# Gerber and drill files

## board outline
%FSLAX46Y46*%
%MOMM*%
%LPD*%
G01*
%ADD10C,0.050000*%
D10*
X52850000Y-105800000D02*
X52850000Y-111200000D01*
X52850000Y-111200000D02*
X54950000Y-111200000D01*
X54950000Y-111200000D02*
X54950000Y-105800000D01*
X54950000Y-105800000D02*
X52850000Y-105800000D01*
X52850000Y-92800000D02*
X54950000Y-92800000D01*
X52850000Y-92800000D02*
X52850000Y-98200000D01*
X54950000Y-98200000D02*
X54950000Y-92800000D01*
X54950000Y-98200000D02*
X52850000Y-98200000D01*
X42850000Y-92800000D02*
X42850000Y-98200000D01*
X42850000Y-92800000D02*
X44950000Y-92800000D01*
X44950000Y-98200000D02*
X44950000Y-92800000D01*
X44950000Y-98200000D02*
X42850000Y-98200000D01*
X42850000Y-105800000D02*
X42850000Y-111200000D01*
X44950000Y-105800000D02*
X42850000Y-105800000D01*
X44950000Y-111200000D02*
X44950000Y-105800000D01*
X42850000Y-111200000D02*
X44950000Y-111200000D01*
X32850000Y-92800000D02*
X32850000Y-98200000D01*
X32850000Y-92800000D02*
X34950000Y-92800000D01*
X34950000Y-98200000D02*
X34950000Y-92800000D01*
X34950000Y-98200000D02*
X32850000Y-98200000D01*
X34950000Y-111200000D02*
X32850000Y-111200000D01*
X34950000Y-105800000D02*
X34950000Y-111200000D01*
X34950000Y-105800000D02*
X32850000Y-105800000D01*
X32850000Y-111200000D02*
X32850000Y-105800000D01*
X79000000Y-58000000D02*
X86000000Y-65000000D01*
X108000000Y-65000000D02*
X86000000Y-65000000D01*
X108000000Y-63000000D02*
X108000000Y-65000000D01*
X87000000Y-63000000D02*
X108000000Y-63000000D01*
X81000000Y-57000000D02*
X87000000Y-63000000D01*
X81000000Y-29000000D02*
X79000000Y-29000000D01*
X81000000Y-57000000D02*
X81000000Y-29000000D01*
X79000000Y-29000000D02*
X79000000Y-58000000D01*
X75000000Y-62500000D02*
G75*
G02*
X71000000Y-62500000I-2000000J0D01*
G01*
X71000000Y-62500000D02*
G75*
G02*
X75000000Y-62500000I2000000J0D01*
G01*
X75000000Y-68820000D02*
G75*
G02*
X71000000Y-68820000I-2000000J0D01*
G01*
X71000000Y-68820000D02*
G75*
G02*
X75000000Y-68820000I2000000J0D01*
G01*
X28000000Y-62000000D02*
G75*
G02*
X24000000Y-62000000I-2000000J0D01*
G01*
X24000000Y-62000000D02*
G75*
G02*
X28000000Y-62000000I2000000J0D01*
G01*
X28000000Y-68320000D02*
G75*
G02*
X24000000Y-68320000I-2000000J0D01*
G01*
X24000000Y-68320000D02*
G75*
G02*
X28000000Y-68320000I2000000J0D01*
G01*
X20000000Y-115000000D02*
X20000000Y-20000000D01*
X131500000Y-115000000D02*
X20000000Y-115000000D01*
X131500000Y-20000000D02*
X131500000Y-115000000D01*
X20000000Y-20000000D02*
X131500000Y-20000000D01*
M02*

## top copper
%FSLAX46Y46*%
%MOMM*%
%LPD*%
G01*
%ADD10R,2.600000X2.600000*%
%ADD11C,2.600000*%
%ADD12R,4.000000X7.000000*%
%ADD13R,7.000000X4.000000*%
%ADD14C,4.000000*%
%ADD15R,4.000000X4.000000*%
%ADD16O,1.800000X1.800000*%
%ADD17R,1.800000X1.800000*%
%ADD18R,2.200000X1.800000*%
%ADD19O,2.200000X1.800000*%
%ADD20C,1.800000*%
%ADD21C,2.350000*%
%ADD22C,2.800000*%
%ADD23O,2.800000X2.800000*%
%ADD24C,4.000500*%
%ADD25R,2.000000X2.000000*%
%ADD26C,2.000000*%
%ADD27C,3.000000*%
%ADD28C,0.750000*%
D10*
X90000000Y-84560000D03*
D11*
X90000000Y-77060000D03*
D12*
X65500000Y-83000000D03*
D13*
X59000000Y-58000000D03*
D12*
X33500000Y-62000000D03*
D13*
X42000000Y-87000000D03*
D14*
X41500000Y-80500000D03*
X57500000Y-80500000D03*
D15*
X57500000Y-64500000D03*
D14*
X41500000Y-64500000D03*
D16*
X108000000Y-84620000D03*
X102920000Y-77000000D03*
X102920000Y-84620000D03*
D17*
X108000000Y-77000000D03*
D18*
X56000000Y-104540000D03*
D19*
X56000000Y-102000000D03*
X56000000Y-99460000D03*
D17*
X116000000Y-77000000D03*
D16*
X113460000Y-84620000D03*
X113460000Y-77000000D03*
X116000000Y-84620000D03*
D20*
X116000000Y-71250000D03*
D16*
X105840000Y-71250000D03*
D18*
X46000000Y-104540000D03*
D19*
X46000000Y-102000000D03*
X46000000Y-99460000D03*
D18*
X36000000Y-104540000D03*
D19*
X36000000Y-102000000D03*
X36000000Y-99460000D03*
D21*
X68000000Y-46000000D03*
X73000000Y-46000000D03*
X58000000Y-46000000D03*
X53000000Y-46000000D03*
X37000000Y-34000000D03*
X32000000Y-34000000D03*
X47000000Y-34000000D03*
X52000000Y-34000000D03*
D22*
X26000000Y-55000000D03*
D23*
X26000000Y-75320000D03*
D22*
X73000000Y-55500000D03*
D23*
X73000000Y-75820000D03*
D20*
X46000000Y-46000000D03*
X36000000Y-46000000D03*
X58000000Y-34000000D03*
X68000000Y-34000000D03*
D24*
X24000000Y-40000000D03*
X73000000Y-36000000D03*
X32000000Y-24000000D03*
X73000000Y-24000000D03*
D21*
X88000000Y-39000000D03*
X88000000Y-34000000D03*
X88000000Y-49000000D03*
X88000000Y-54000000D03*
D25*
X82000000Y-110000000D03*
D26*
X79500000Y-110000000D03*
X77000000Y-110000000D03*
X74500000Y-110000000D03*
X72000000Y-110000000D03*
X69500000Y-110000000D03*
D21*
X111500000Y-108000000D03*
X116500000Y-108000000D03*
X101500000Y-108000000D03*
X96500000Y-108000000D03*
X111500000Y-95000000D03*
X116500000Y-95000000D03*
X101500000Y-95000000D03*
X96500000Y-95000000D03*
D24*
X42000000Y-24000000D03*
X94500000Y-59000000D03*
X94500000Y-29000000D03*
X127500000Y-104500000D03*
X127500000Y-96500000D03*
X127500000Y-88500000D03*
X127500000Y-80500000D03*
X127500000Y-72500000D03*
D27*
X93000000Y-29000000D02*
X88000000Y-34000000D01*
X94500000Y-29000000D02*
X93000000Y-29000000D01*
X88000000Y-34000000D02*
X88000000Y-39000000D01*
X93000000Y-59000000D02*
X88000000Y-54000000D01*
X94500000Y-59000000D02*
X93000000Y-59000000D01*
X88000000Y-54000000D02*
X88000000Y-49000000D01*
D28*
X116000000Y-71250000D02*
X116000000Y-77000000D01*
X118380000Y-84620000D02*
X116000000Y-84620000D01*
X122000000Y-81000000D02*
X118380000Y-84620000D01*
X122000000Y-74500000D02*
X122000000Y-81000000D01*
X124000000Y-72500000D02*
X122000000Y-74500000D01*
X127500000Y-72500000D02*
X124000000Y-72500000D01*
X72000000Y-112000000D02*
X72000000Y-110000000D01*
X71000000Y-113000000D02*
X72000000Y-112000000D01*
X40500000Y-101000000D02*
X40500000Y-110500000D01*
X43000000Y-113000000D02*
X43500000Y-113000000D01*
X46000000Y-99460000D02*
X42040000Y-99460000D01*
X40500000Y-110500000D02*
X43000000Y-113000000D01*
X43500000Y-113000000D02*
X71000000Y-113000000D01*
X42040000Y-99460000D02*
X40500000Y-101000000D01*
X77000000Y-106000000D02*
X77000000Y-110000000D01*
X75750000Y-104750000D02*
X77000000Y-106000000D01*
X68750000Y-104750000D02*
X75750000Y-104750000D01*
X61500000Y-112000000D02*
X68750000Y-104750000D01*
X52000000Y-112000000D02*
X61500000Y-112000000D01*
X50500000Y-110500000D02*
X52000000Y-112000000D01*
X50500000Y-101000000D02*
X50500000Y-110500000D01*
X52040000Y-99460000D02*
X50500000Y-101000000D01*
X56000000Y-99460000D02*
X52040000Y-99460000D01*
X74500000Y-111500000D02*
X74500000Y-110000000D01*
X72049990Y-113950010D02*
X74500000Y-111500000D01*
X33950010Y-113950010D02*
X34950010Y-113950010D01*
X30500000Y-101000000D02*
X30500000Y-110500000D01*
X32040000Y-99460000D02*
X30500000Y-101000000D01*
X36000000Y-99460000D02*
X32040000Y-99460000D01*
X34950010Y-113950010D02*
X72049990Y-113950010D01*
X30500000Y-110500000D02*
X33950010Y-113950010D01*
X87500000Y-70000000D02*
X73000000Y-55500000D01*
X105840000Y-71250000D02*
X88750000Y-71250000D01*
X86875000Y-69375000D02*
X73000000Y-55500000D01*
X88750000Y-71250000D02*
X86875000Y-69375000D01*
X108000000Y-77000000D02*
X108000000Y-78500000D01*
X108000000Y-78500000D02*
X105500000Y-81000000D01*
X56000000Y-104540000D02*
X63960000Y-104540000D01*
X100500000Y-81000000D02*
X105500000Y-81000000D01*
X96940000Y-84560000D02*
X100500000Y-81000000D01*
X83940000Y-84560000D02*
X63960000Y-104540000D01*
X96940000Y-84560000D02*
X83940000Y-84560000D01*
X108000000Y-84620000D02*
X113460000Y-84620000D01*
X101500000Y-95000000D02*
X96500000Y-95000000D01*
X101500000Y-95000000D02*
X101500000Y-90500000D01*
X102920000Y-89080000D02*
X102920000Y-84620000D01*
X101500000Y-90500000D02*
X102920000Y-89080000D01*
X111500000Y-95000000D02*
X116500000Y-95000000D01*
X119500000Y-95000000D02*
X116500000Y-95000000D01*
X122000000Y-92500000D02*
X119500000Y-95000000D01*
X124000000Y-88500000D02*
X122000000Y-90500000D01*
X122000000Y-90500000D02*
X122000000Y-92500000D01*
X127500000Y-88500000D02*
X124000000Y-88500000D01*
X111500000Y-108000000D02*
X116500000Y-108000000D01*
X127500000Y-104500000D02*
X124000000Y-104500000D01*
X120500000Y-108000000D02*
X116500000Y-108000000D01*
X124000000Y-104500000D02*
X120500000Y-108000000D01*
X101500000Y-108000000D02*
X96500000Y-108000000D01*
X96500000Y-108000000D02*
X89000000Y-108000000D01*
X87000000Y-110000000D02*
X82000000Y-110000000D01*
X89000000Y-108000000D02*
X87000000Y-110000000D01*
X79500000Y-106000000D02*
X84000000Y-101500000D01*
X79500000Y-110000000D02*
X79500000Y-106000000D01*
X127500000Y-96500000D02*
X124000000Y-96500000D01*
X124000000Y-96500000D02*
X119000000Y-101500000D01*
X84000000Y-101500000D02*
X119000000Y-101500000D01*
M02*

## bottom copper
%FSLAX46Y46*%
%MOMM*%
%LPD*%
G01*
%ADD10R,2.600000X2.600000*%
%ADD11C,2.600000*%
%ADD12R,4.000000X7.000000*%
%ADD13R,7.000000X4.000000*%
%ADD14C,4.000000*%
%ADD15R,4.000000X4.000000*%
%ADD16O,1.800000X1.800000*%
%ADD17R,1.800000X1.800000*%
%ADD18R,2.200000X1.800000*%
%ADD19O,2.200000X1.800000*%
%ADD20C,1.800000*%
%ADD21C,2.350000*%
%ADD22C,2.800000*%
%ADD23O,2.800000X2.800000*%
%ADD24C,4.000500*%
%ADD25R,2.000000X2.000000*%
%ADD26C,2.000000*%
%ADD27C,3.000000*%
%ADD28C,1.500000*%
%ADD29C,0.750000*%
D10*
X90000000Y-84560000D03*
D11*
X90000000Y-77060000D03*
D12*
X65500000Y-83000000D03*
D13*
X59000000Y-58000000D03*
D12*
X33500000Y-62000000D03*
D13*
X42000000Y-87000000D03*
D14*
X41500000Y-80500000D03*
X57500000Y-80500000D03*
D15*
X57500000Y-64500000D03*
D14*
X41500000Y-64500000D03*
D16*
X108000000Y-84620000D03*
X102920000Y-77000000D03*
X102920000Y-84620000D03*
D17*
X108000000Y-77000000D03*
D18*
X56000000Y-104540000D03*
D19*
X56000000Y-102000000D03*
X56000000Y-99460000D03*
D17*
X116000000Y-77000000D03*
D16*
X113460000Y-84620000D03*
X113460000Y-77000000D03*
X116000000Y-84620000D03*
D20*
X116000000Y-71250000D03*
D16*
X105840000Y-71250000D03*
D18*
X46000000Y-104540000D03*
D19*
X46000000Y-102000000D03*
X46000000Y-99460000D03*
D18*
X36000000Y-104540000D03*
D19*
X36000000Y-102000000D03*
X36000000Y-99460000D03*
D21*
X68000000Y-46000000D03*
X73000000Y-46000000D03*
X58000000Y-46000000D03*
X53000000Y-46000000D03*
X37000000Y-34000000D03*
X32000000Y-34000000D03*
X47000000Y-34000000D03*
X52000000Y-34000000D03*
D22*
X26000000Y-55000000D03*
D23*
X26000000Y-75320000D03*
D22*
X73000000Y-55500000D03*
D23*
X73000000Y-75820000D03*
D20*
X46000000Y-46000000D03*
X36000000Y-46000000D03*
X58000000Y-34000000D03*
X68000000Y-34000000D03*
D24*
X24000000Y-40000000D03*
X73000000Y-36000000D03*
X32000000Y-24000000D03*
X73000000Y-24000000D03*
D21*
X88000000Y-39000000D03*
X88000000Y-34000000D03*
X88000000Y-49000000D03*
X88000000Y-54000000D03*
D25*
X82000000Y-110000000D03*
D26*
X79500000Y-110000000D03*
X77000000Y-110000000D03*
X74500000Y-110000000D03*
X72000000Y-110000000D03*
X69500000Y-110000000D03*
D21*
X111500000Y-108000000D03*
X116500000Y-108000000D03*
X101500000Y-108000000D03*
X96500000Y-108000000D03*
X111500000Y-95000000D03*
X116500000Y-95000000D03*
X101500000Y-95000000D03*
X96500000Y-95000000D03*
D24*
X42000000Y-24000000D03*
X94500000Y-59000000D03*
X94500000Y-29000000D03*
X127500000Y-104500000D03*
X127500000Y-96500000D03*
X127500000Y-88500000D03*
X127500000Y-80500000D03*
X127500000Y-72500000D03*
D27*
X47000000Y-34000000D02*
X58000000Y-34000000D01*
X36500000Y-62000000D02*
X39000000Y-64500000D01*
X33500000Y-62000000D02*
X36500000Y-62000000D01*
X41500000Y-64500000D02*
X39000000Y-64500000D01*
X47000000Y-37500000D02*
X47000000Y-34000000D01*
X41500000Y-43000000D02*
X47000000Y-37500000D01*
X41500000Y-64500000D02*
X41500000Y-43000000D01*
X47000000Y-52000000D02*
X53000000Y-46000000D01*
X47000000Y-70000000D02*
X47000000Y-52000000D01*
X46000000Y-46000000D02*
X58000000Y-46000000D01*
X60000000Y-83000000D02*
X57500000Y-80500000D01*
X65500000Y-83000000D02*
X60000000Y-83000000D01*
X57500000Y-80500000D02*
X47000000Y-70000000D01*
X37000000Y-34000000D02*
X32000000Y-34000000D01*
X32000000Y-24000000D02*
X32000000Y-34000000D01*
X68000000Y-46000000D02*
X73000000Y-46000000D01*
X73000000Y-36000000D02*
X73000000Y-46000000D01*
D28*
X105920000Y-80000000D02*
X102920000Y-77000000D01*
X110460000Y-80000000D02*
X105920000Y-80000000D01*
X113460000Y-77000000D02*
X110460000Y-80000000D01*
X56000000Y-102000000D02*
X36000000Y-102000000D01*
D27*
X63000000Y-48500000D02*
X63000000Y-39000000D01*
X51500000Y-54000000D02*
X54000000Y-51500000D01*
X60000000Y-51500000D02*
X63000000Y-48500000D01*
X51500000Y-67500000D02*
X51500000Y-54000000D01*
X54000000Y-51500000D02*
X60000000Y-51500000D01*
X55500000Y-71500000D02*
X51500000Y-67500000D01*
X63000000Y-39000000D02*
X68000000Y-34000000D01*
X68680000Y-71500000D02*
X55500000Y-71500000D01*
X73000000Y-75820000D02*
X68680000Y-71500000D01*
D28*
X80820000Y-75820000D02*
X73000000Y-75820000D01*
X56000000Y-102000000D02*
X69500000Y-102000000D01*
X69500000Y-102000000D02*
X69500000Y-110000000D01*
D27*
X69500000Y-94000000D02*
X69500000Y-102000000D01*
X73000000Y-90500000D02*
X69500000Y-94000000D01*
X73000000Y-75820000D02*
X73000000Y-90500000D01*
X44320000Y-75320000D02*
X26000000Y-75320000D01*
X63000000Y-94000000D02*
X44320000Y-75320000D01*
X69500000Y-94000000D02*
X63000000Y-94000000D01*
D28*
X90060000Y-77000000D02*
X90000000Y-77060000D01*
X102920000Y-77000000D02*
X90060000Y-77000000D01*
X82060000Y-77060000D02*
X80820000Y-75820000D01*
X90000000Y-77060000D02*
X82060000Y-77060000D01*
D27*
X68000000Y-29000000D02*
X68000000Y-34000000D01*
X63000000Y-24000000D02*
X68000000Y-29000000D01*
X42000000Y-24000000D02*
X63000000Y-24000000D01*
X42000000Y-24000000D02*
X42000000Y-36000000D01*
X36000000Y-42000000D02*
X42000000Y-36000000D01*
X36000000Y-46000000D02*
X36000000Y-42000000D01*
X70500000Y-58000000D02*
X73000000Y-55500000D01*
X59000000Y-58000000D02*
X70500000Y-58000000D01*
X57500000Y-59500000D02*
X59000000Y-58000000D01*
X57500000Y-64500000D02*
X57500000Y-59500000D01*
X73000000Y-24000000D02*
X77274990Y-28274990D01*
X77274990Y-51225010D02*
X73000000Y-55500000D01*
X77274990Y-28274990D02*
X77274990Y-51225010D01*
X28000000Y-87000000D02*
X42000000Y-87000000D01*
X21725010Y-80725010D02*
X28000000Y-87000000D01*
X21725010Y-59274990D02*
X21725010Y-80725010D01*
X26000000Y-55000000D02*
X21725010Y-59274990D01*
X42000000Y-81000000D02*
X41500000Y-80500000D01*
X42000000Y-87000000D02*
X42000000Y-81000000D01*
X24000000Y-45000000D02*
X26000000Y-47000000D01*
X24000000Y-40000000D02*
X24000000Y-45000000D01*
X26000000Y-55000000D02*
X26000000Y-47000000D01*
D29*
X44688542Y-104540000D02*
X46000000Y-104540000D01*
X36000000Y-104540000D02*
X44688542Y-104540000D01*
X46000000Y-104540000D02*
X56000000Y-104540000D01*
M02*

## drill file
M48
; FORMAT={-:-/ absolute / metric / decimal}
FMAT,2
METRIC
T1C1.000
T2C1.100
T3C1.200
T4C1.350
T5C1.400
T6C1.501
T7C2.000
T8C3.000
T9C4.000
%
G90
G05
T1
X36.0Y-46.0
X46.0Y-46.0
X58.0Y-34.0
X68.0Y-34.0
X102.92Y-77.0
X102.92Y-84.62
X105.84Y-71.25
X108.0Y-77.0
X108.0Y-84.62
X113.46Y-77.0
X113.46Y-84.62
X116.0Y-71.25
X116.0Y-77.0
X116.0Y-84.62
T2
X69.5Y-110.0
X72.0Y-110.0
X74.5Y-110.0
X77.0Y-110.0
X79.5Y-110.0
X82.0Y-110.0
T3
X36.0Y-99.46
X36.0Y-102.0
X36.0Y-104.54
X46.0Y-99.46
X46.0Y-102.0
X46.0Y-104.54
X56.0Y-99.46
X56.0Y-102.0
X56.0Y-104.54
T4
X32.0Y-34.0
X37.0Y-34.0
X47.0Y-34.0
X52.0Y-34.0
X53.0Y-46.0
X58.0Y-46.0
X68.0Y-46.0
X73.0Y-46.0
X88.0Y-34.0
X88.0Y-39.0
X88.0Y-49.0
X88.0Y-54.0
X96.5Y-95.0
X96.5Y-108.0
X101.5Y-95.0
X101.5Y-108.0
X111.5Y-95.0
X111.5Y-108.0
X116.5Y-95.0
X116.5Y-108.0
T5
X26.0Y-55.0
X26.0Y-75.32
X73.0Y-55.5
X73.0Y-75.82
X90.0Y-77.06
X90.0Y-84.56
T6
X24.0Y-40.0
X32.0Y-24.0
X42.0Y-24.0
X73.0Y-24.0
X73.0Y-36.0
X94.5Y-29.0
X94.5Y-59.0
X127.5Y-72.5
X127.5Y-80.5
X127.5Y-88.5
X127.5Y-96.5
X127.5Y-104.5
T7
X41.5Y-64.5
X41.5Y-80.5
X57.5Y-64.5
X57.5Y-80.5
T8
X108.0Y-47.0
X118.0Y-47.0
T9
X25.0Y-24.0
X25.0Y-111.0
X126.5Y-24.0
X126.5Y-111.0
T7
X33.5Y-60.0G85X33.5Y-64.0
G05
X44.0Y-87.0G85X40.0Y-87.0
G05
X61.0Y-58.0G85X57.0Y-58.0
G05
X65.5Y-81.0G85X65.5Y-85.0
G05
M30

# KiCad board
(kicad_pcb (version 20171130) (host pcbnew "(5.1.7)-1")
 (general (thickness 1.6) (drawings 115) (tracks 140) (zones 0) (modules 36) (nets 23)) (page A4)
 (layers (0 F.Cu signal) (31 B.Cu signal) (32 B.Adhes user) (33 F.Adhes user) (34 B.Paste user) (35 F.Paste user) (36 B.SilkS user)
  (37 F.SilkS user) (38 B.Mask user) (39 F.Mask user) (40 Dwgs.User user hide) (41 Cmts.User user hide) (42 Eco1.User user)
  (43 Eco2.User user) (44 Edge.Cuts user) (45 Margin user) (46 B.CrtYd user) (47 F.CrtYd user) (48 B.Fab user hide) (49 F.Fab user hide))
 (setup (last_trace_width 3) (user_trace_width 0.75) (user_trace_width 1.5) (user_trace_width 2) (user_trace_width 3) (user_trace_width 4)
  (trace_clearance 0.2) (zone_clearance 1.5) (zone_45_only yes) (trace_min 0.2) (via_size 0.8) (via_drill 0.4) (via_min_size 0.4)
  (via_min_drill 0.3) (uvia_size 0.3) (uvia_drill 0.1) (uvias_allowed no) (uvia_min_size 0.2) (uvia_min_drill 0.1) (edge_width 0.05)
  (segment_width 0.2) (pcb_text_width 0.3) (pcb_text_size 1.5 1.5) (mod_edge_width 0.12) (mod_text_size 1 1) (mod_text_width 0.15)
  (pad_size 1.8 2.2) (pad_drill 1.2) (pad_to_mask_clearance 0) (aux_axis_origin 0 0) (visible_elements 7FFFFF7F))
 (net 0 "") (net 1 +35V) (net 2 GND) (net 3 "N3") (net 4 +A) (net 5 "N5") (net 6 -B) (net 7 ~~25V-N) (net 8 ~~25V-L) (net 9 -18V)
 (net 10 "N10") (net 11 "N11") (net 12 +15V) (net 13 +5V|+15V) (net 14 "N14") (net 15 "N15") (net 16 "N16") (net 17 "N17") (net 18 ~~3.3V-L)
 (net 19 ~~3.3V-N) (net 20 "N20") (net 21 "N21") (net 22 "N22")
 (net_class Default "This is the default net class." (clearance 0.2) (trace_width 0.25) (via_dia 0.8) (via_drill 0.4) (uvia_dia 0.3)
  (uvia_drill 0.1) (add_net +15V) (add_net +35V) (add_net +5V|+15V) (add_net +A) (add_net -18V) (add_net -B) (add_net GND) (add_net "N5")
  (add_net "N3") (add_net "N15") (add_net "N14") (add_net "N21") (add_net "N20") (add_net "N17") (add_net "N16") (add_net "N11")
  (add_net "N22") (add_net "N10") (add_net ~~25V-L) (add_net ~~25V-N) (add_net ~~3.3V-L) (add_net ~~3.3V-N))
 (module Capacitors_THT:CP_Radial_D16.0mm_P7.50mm (layer F.Cu) (at 90 84.56 90)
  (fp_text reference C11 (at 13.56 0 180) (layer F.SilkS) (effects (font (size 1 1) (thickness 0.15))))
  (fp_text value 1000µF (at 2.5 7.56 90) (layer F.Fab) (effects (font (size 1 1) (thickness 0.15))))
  (pad 1 thru_hole rect (at 0 0 90) (size 2.6 2.6) (drill 1.4) (layers *.Cu *.Mask) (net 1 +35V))
  (pad 2 thru_hole circle (at 7.5 0 90) (size 2.6 2.6) (drill 1.4) (layers *.Cu *.Mask) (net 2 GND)))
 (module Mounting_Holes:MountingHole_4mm (layer F.Cu) (at 126.5 24)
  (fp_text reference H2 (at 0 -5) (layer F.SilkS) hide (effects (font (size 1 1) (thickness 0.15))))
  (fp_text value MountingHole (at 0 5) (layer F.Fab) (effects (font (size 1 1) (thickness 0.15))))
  (pad 1 np_thru_hole circle (at 0 0) (size 4 4) (drill 4) (layers *.Cu *.Mask)))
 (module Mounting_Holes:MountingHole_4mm (layer F.Cu) (at 25 24)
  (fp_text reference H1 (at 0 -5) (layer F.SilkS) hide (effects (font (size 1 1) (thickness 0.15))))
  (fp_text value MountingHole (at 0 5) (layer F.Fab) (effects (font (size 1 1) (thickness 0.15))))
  (pad 1 np_thru_hole circle (at 0 0) (size 4 4) (drill 4) (layers *.Cu *.Mask)))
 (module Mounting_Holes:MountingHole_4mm (layer F.Cu) (at 25 111)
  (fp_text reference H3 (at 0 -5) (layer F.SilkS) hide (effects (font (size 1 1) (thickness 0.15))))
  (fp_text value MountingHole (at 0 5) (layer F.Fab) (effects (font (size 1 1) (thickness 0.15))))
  (pad 1 np_thru_hole circle (at 0 0) (size 4 4) (drill 4) (layers *.Cu *.Mask)))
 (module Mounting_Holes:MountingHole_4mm (layer F.Cu) (at 126.5 111)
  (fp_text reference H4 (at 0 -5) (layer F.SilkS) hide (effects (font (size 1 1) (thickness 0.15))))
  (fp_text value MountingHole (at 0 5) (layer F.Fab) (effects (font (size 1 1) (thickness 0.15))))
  (pad 1 np_thru_hole circle (at 0 0) (size 4 4) (drill 4) (layers *.Cu *.Mask)))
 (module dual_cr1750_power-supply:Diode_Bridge (layer F.Cu) (at 32 90 90)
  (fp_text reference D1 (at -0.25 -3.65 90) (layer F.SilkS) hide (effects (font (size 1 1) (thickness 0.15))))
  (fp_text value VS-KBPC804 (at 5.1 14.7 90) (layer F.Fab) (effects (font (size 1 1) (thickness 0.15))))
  (pad 2 thru_hole rect (at 7 33.5 270) (size 7 4) (drill oval 6 2) (layers B.Cu B.Mask) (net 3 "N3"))
  (pad 3 thru_hole rect (at 32 27 180) (size 7 4) (drill oval 6 2) (layers B.Cu B.Mask) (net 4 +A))
  (pad 4 thru_hole rect (at 28 1.5 270) (size 7 4) (drill oval 6 2) (layers B.Cu B.Mask) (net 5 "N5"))
  (pad 1 thru_hole rect (at 3 10 180) (size 7 4) (drill oval 6 2) (layers B.Cu B.Mask) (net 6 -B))
  (pad 1 thru_hole circle (at 9.5 9.5 90) (size 4 4) (drill 2) (layers B.Cu B.Mask) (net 6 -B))
  (pad 2 thru_hole circle (at 9.5 25.5 90) (size 4 4) (drill 2) (layers B.Cu B.Mask) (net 3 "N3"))
  (pad 3 thru_hole rect (at 25.5 25.5 90) (size 4 4) (drill 2) (layers B.Cu B.Mask) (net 4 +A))
  (pad 4 thru_hole circle (at 25.5 9.5 90) (size 4 4) (drill 2) (layers B.Cu B.Mask) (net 5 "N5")))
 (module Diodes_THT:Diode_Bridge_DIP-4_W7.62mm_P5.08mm (layer F.Cu) (at 108 77 270)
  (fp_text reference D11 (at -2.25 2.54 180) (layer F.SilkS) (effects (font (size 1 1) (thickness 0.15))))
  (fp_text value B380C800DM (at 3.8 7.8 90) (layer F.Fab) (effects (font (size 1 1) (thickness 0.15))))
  (pad 4 thru_hole oval (at 7.62 0 270) (size 1.8 1.8) (drill 1) (layers *.Cu *.Mask) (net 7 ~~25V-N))
  (pad 2 thru_hole oval (at 0 5.08 270) (size 1.8 1.8) (drill 1) (layers *.Cu *.Mask) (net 2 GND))
  (pad 3 thru_hole oval (at 7.62 5.08 270) (size 1.8 1.8) (drill 1) (layers *.Cu *.Mask) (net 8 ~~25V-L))
  (pad 1 thru_hole rect (at 0 0 270) (size 1.8 1.8) (drill 1) (layers *.Cu *.Mask) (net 1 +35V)))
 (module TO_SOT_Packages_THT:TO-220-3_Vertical (layer F.Cu) (at 56 104.54 90)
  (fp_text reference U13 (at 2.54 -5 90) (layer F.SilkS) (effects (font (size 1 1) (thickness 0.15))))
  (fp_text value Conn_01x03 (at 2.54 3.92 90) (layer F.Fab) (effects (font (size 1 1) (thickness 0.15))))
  (pad 1 thru_hole rect (at 0 0 90) (size 1.8 2.2) (drill 1.2) (layers *.Cu *.Mask) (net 1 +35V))
  (pad 2 thru_hole oval (at 2.54 0 90) (size 1.8 2.2) (drill 1.2) (layers *.Cu *.Mask) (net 2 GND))
  (pad 3 thru_hole oval (at 5.08 0 90) (size 1.8 2.2) (drill 1.2) (layers *.Cu *.Mask) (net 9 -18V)))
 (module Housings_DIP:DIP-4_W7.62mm (layer F.Cu) (at 116 77 270)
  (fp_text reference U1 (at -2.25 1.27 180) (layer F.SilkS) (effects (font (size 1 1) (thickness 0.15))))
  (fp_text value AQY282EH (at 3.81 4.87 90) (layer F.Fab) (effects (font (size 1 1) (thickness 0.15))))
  (pad 1 thru_hole rect (at 0 0 270) (size 1.8 1.8) (drill 1) (layers *.Cu *.Mask) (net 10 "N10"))
  (pad 3 thru_hole oval (at 7.62 2.54 270) (size 1.8 1.8) (drill 1) (layers *.Cu *.Mask) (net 7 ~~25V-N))
  (pad 2 thru_hole oval (at 0 2.54 270) (size 1.8 1.8) (drill 1) (layers *.Cu *.Mask) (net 2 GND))
  (pad 4 thru_hole oval (at 7.62 0 270) (size 1.8 1.8) (drill 1) (layers *.Cu *.Mask) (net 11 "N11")))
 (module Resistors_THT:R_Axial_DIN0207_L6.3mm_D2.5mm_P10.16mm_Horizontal (layer F.Cu) (at 116 71.25 180)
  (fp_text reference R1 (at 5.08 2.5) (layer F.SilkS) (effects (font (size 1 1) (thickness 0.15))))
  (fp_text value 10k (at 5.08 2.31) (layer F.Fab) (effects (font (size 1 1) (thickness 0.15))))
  (pad 1 thru_hole circle (at 0 0 180) (size 1.8 1.8) (drill 1) (layers *.Cu *.Mask) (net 10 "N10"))
  (pad 2 thru_hole oval (at 10.16 0 180) (size 1.8 1.8) (drill 1) (layers *.Cu *.Mask) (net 4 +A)))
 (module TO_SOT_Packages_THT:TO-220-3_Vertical (layer F.Cu) (at 46 104.54 90)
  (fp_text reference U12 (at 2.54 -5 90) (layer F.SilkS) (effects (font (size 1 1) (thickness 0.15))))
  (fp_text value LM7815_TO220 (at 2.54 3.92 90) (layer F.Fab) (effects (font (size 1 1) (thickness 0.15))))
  (pad 1 thru_hole rect (at 0 0 90) (size 1.8 2.2) (drill 1.2) (layers *.Cu *.Mask) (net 1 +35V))
  (pad 2 thru_hole oval (at 2.54 0 90) (size 1.8 2.2) (drill 1.2) (layers *.Cu *.Mask) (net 2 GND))
  (pad 3 thru_hole oval (at 5.08 0 90) (size 1.8 2.2) (drill 1.2) (layers *.Cu *.Mask) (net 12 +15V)))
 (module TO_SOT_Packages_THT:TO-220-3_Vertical (layer F.Cu) (at 36 104.54 90)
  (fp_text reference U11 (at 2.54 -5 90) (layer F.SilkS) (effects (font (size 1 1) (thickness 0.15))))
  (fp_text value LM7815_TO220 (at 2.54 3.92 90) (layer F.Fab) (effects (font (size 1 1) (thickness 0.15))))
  (pad 1 thru_hole rect (at 0 0 90) (size 1.8 2.2) (drill 1.2) (layers *.Cu *.Mask) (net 1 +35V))
  (pad 2 thru_hole oval (at 2.54 0 90) (size 1.8 2.2) (drill 1.2) (layers *.Cu *.Mask) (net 2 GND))
  (pad 3 thru_hole oval (at 5.08 0 90) (size 1.8 2.2) (drill 1.2) (layers *.Cu *.Mask) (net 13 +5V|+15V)))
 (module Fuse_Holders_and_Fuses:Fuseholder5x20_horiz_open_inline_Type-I (layer F.Cu) (at 53 46)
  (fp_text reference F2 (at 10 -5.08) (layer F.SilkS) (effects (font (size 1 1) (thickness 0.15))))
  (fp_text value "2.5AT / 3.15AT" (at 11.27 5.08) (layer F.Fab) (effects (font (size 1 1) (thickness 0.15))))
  (pad 2 thru_hole circle (at 15 0) (size 2.35 2.35) (drill 1.35) (layers *.Cu *.Mask) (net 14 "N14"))
  (pad 2 thru_hole circle (at 20 0) (size 2.35 2.35) (drill 1.35) (layers *.Cu *.Mask) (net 14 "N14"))
  (pad 1 thru_hole circle (at 5 0) (size 2.35 2.35) (drill 1.35) (layers *.Cu *.Mask) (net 3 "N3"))
  (pad 1 thru_hole circle (at 0 0) (size 2.35 2.35) (drill 1.35) (layers *.Cu *.Mask) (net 3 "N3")))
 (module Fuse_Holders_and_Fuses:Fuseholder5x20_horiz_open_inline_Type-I (layer F.Cu) (at 52 34 180)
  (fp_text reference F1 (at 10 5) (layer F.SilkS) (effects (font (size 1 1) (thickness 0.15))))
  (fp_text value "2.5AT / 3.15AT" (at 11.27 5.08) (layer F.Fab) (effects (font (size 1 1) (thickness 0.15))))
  (pad 2 thru_hole circle (at 15 0 180) (size 2.35 2.35) (drill 1.35) (layers *.Cu *.Mask) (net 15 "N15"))
  (pad 2 thru_hole circle (at 20 0 180) (size 2.35 2.35) (drill 1.35) (layers *.Cu *.Mask) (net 15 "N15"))
  (pad 1 thru_hole circle (at 5 0 180) (size 2.35 2.35) (drill 1.35) (layers *.Cu *.Mask) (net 5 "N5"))
  (pad 1 thru_hole circle (at 0 0 180) (size 2.35 2.35) (drill 1.35) (layers *.Cu *.Mask) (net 5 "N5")))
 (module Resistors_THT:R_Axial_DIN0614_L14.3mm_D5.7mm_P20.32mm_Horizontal (layer F.Cu) (at 26 55 270)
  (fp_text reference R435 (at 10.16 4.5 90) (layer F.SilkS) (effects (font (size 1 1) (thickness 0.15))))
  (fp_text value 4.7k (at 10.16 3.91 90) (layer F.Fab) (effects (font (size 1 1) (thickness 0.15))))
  (pad 1 thru_hole circle (at 0 0 270) (size 2.8 2.8) (drill 1.4) (layers *.Cu *.Mask) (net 6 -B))
  (pad 2 thru_hole oval (at 20.32 0 270) (size 2.8 2.8) (drill 1.4) (layers *.Cu *.Mask) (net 2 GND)))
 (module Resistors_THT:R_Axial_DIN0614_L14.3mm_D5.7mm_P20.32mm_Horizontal (layer F.Cu) (at 73 55.5 270)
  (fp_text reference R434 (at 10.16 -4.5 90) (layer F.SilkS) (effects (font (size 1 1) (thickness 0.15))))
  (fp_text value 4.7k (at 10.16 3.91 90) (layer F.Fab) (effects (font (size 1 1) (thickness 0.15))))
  (pad 1 thru_hole circle (at 0 0 270) (size 2.8 2.8) (drill 1.4) (layers *.Cu *.Mask) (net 4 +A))
  (pad 2 thru_hole oval (at 20.32 0 270) (size 2.8 2.8) (drill 1.4) (layers *.Cu *.Mask) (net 2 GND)))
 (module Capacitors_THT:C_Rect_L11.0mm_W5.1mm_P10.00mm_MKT (layer F.Cu) (at 46 46 180)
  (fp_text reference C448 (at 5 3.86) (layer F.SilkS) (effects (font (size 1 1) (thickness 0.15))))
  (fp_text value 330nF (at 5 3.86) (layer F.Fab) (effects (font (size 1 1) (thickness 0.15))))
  (pad 1 thru_hole circle (at 0 0 180) (size 1.8 1.8) (drill 1) (layers *.Cu *.Mask) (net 3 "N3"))
  (pad 2 thru_hole circle (at 10 0 180) (size 1.8 1.8) (drill 1) (layers *.Cu *.Mask) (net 2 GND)))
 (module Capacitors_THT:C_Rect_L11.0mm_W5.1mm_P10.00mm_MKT (layer F.Cu) (at 58 34)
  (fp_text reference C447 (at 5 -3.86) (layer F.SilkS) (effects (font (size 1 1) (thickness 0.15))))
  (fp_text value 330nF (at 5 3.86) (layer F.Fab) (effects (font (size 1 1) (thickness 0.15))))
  (pad 1 thru_hole circle (at 0 0) (size 1.8 1.8) (drill 1) (layers *.Cu *.Mask) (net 5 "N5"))
  (pad 2 thru_hole circle (at 10 0) (size 1.8 1.8) (drill 1) (layers *.Cu *.Mask) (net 2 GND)))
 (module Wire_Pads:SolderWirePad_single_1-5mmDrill (layer F.Cu) (at 24 40)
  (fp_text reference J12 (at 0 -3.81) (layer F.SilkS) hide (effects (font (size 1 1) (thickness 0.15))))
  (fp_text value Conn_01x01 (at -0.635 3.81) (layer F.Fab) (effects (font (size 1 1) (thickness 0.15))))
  (pad 1 thru_hole circle (at 0 0) (size 4.0005 4.0005) (drill 1.50114) (layers *.Cu *.Mask) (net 6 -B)))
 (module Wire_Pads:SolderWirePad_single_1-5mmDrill (layer F.Cu) (at 73 36)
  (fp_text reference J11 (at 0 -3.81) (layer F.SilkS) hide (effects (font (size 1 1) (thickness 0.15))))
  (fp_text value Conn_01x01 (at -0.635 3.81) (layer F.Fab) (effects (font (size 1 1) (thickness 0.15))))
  (pad 1 thru_hole circle (at 0 0) (size 4.0005 4.0005) (drill 1.50114) (layers *.Cu *.Mask) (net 14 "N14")))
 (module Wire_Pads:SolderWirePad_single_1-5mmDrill (layer F.Cu) (at 32 24)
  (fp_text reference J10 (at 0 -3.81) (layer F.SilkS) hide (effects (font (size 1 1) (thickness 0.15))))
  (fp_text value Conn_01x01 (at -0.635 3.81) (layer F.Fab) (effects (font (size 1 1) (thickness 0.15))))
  (pad 1 thru_hole circle (at 0 0) (size 4.0005 4.0005) (drill 1.50114) (layers *.Cu *.Mask) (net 15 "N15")))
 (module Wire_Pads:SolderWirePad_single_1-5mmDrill (layer F.Cu) (at 73 24)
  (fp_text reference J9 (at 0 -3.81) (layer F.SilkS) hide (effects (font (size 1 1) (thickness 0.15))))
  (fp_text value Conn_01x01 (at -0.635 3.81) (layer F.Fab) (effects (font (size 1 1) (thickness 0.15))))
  (pad 1 thru_hole circle (at 0 0) (size 4.0005 4.0005) (drill 1.50114) (layers *.Cu *.Mask) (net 4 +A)))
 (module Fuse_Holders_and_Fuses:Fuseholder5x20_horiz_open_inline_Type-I (layer F.Cu) (at 88 54 90)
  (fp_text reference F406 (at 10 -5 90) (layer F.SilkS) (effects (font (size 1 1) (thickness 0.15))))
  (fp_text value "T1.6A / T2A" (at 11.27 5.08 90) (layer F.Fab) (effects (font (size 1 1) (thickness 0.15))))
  (pad 2 thru_hole circle (at 15 0 90) (size 2.35 2.35) (drill 1.35) (layers *.Cu *.Mask) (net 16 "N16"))
  (pad 2 thru_hole circle (at 20 0 90) (size 2.35 2.35) (drill 1.35) (layers *.Cu *.Mask) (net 16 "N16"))
  (pad 1 thru_hole circle (at 5 0 90) (size 2.35 2.35) (drill 1.35) (layers *.Cu *.Mask) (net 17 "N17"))
  (pad 1 thru_hole circle (at 0 0 90) (size 2.35 2.35) (drill 1.35) (layers *.Cu *.Mask) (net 17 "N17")))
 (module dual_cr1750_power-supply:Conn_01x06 (layer F.Cu) (at 82 110 180) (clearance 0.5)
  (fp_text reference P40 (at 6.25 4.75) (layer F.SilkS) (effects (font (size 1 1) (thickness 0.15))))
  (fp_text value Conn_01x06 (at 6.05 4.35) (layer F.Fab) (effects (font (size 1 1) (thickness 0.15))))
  (pad 1 thru_hole rect (at 0 0 180) (size 2 2) (drill 1.1) (layers *.Cu *.Mask) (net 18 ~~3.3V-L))
  (pad 2 thru_hole circle (at 2.5 0 180) (size 2 2) (drill 1.1) (layers *.Cu *.Mask) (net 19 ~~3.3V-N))
  (pad 3 thru_hole circle (at 5 0 180) (size 2 2) (drill 1.1) (layers *.Cu *.Mask) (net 9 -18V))
  (pad 4 thru_hole circle (at 7.5 0 180) (size 2 2) (drill 1.1) (layers *.Cu *.Mask) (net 13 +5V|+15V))
  (pad 5 thru_hole circle (at 10 0 180) (size 2 2) (drill 1.1) (layers *.Cu *.Mask) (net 12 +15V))
  (pad 6 thru_hole circle (at 12.5 0 180) (size 2 2) (drill 1.1) (layers *.Cu *.Mask) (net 2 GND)))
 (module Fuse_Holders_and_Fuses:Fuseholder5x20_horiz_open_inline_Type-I (layer F.Cu) (at 96.5 108)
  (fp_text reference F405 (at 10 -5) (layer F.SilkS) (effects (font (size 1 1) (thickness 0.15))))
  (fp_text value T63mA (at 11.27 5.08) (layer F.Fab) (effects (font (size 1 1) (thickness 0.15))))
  (pad 2 thru_hole circle (at 15 0) (size 2.35 2.35) (drill 1.35) (layers *.Cu *.Mask) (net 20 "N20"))
  (pad 2 thru_hole circle (at 20 0) (size 2.35 2.35) (drill 1.35) (layers *.Cu *.Mask) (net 20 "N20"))
  (pad 1 thru_hole circle (at 5 0) (size 2.35 2.35) (drill 1.35) (layers *.Cu *.Mask) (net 18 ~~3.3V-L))
  (pad 1 thru_hole circle (at 0 0) (size 2.35 2.35) (drill 1.35) (layers *.Cu *.Mask) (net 18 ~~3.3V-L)))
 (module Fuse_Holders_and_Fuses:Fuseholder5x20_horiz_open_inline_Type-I (layer F.Cu) (at 96.5 95)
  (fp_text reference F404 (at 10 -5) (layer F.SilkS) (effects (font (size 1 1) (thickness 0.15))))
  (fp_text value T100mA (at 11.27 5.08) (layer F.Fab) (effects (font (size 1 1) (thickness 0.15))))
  (pad 2 thru_hole circle (at 15 0) (size 2.35 2.35) (drill 1.35) (layers *.Cu *.Mask) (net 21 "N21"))
  (pad 2 thru_hole circle (at 20 0) (size 2.35 2.35) (drill 1.35) (layers *.Cu *.Mask) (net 21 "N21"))
  (pad 1 thru_hole circle (at 5 0) (size 2.35 2.35) (drill 1.35) (layers *.Cu *.Mask) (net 8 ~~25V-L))
  (pad 1 thru_hole circle (at 0 0) (size 2.35 2.35) (drill 1.35) (layers *.Cu *.Mask) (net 8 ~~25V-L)))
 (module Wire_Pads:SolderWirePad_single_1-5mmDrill (layer F.Cu) (at 42 24)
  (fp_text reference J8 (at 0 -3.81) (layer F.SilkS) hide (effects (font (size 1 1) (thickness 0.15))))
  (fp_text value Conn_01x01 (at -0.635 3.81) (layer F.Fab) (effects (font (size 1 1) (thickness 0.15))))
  (pad 1 thru_hole circle (at 0 0) (size 4.0005 4.0005) (drill 1.50114) (layers *.Cu *.Mask) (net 2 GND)))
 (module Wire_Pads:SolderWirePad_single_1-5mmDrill (layer F.Cu) (at 94.5 59)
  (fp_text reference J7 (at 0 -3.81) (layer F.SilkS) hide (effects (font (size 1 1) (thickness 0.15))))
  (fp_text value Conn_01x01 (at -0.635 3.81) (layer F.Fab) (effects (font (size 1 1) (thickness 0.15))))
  (pad 1 thru_hole circle (at 0 0) (size 4.0005 4.0005) (drill 1.50114) (layers *.Cu *.Mask) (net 17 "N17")))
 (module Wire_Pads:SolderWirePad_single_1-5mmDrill (layer F.Cu) (at 94.5 29)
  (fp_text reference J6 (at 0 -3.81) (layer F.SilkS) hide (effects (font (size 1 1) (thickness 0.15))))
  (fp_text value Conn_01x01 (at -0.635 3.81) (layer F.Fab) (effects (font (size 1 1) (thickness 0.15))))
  (pad 1 thru_hole circle (at 0 0) (size 4.0005 4.0005) (drill 1.50114) (layers *.Cu *.Mask) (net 16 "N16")))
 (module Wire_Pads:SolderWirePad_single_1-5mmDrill (layer F.Cu) (at 127.5 104.5)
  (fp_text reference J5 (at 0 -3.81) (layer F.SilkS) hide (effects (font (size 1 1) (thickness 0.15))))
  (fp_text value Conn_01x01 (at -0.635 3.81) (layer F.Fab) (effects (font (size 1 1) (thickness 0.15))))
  (pad 1 thru_hole circle (at 0 0) (size 4.0005 4.0005) (drill 1.50114) (layers *.Cu *.Mask) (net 20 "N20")))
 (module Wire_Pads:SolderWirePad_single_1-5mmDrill (layer F.Cu) (at 127.5 96.5)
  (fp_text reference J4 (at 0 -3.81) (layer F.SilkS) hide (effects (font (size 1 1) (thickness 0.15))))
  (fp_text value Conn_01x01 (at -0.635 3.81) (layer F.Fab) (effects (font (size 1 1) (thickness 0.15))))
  (pad 1 thru_hole circle (at 0 0) (size 4.0005 4.0005) (drill 1.50114) (layers *.Cu *.Mask) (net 19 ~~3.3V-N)))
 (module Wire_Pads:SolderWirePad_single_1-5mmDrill (layer F.Cu) (at 127.5 88.5)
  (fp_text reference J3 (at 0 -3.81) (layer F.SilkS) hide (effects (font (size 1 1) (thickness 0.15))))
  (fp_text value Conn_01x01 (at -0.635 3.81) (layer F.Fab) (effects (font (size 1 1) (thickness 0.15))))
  (pad 1 thru_hole circle (at 0 0) (size 4.0005 4.0005) (drill 1.50114) (layers *.Cu *.Mask) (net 21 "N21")))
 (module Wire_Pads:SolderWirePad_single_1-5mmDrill (layer F.Cu) (at 127.5 80.5)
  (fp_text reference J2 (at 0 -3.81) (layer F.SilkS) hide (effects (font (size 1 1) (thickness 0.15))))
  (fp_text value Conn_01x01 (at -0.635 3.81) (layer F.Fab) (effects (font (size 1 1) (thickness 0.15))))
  (pad 1 thru_hole circle (at 0 0) (size 4.0005 4.0005) (drill 1.50114) (layers *.Cu *.Mask) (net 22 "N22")))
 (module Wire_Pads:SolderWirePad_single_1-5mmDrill (layer F.Cu) (at 127.5 72.5)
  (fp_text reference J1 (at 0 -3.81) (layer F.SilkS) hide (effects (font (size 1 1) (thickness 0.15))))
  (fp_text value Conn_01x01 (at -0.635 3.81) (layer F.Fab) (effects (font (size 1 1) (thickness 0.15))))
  (pad 1 thru_hole circle (at 0 0) (size 4.0005 4.0005) (drill 1.50114) (layers *.Cu *.Mask) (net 11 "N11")))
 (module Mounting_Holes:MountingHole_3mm (layer F.Cu) (at 118 47)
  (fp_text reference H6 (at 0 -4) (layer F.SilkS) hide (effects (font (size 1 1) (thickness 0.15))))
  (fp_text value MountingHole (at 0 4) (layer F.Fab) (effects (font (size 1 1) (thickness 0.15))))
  (pad 1 np_thru_hole circle (at 0 0) (size 3 3) (drill 3) (layers *.Cu *.Mask)))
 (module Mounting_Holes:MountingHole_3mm (layer F.Cu) (at 108 47)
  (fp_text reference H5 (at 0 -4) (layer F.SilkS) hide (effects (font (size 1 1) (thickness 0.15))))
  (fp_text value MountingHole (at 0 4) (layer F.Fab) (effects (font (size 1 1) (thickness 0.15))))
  (pad 1 np_thru_hole circle (at 0 0) (size 3 3) (drill 3) (layers *.Cu *.Mask)))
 (gr_line (start 52.85 105.8) (end 52.85 111.2) (layer Edge.Cuts) (width 0.05))
 (gr_line (start 52.85 111.2) (end 54.95 111.2) (layer Edge.Cuts) (width 0.05))
 (gr_line (start 54.95 111.2) (end 54.95 105.8) (layer Edge.Cuts) (width 0.05))
 (gr_line (start 54.95 105.8) (end 52.85 105.8) (layer Edge.Cuts) (width 0.05))
 (gr_line (start 52.85 92.8) (end 54.95 92.8) (layer Edge.Cuts) (width 0.05))
 (gr_line (start 52.85 92.8) (end 52.85 98.2) (layer Edge.Cuts) (width 0.05))
 (gr_line (start 54.95 98.2) (end 54.95 92.8) (layer Edge.Cuts) (width 0.05))
 (gr_line (start 54.95 98.2) (end 52.85 98.2) (layer Edge.Cuts) (width 0.05))
 (gr_line (start 42.85 92.8) (end 42.85 98.2) (layer Edge.Cuts) (width 0.05))
 (gr_line (start 42.85 92.8) (end 44.95 92.8) (layer Edge.Cuts) (width 0.05))
 (gr_line (start 44.95 98.2) (end 44.95 92.8) (layer Edge.Cuts) (width 0.05))
 (gr_line (start 44.95 98.2) (end 42.85 98.2) (layer Edge.Cuts) (width 0.05))
 (gr_line (start 42.85 105.8) (end 42.85 111.2) (layer Edge.Cuts) (width 0.05))
 (gr_line (start 44.95 105.8) (end 42.85 105.8) (layer Edge.Cuts) (width 0.05))
 (gr_line (start 44.95 111.2) (end 44.95 105.8) (layer Edge.Cuts) (width 0.05))
 (gr_line (start 42.85 111.2) (end 44.95 111.2) (layer Edge.Cuts) (width 0.05))
 (gr_line (start 32.85 92.8) (end 32.85 98.2) (layer Edge.Cuts) (width 0.05))
 (gr_line (start 32.85 92.8) (end 34.95 92.8) (layer Edge.Cuts) (width 0.05))
 (gr_line (start 34.95 98.2) (end 34.95 92.8) (layer Edge.Cuts) (width 0.05))
 (gr_line (start 34.95 98.2) (end 32.85 98.2) (layer Edge.Cuts) (width 0.05))
 (gr_line (start 34.95 111.2) (end 32.85 111.2) (layer Edge.Cuts) (width 0.05))
 (gr_line (start 34.95 105.8) (end 34.95 111.2) (layer Edge.Cuts) (width 0.05))
 (gr_line (start 34.95 105.8) (end 32.85 105.8) (layer Edge.Cuts) (width 0.05))
 (gr_line (start 32.85 111.2) (end 32.85 105.8) (layer Edge.Cuts) (width 0.05))
 (gr_line (start 79 58) (end 86 65) (layer Edge.Cuts) (width 0.05))
 (gr_line (start 108 65) (end 86 65) (layer Edge.Cuts) (width 0.05))
 (gr_line (start 108 63) (end 108 65) (layer Edge.Cuts) (width 0.05))
 (gr_line (start 87 63) (end 108 63) (layer Edge.Cuts) (width 0.05))
 (gr_line (start 81 57) (end 87 63) (layer Edge.Cuts) (width 0.05))
 (gr_line (start 81 29) (end 79 29) (layer Edge.Cuts) (width 0.05))
 (gr_line (start 81 57) (end 81 29) (layer Edge.Cuts) (width 0.05))
 (gr_line (start 79 29) (end 79 58) (layer Edge.Cuts) (width 0.05))
 (gr_circle (center 73 62.5) (end 73 60.5) (layer Edge.Cuts) (width 0.05))
 (gr_circle (center 73 68.82) (end 73 66.82) (layer Edge.Cuts) (width 0.05))
 (gr_circle (center 26 62) (end 28 62) (layer Edge.Cuts) (width 0.05))
 (gr_circle (center 26 68.32) (end 28 68.32) (layer Edge.Cuts) (width 0.05))
 (gr_line (start 20 115) (end 20 20) (layer Edge.Cuts) (width 0.05))
 (gr_line (start 131.5 115) (end 20 115) (layer Edge.Cuts) (width 0.05))
 (gr_line (start 131.5 20) (end 131.5 115) (layer Edge.Cuts) (width 0.05))
 (gr_line (start 20 20) (end 131.5 20) (layer Edge.Cuts) (width 0.05))
 (segment (start 93 29) (end 88 34) (width 3) (layer F.Cu) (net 16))
 (segment (start 94.5 29) (end 93 29) (width 3) (layer F.Cu) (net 16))
 (segment (start 88 34) (end 88 39) (width 3) (layer F.Cu) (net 16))
 (segment (start 93 59) (end 88 54) (width 3) (layer F.Cu) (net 17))
 (segment (start 94.5 59) (end 93 59) (width 3) (layer F.Cu) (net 17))
 (segment (start 88 54) (end 88 49) (width 3) (layer F.Cu) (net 17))
 (segment (start 47 34) (end 58 34) (width 3) (layer B.Cu) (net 5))
 (segment (start 36.5 62) (end 39 64.5) (width 3) (layer B.Cu) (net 5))
 (segment (start 33.5 62) (end 36.5 62) (width 3) (layer B.Cu) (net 5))
 (segment (start 41.5 64.5) (end 39 64.5) (width 3) (layer B.Cu) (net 5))
 (segment (start 47 37.5) (end 47 34) (width 3) (layer B.Cu) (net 5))
 (segment (start 41.5 43) (end 47 37.5) (width 3) (layer B.Cu) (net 5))
 (segment (start 41.5 64.5) (end 41.5 43) (width 3) (layer B.Cu) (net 5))
 (segment (start 47 52) (end 53 46) (width 3) (layer B.Cu) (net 3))
 (segment (start 47 70) (end 47 52) (width 3) (layer B.Cu) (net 3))
 (segment (start 46 46) (end 58 46) (width 3) (layer B.Cu) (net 3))
 (segment (start 60 83) (end 57.5 80.5) (width 3) (layer B.Cu) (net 3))
 (segment (start 65.5 83) (end 60 83) (width 3) (layer B.Cu) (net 3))
 (segment (start 57.5 80.5) (end 47 70) (width 3) (layer B.Cu) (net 3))
 (segment (start 37 34) (end 32 34) (width 3) (layer B.Cu) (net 15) (status 1000000))
 (segment (start 32 24) (end 32 34) (width 3) (layer B.Cu) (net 15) (status 1000000))
 (segment (start 68 46) (end 73 46) (width 3) (layer B.Cu) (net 14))
 (segment (start 73 36) (end 73 46) (width 3) (layer B.Cu) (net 14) (status 1000000))
 (segment (start 116 71.25) (end 116 77) (width 0.75) (layer F.Cu) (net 10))
 (segment (start 118.38 84.62) (end 116 84.62) (width 0.75) (layer F.Cu) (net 11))
 (segment (start 122 81) (end 118.38 84.62) (width 0.75) (layer F.Cu) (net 11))
 (segment (start 122 74.5) (end 122 81) (width 0.75) (layer F.Cu) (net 11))
 (segment (start 124 72.5) (end 122 74.5) (width 0.75) (layer F.Cu) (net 11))
 (segment (start 127.5 72.5) (end 124 72.5) (width 0.75) (layer F.Cu) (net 11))
 (segment (start 105.92 80) (end 102.92 77) (width 1.5) (layer B.Cu) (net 2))
 (segment (start 110.46 80) (end 105.92 80) (width 1.5) (layer B.Cu) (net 2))
 (segment (start 113.46 77) (end 110.46 80) (width 1.5) (layer B.Cu) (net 2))
 (segment (start 56 102) (end 36 102) (width 1.5) (layer B.Cu) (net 2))
 (segment (start 63 48.5) (end 63 39) (width 3) (layer B.Cu) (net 2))
 (segment (start 51.5 54) (end 54 51.5) (width 3) (layer B.Cu) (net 2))
 (segment (start 60 51.5) (end 63 48.5) (width 3) (layer B.Cu) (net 2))
 (segment (start 51.5 67.5) (end 51.5 54) (width 3) (layer B.Cu) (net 2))
 (segment (start 54 51.5) (end 60 51.5) (width 3) (layer B.Cu) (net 2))
 (segment (start 55.5 71.5) (end 51.5 67.5) (width 3) (layer B.Cu) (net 2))
 (segment (start 63 39) (end 68 34) (width 3) (layer B.Cu) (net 2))
 (segment (start 68.68 71.5) (end 55.5 71.5) (width 3) (layer B.Cu) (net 2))
 (segment (start 73 75.82) (end 68.68 71.5) (width 3) (layer B.Cu) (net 2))
 (segment (start 80.82 75.82) (end 73 75.82) (width 1.5) (layer B.Cu) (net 2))
 (segment (start 56 102) (end 69.5 102) (width 1.5) (layer B.Cu) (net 2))
 (segment (start 69.5 102) (end 69.5 110) (width 1.5) (layer B.Cu) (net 2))
 (segment (start 69.5 94) (end 69.5 102) (width 3) (layer B.Cu) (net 2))
 (segment (start 73 90.5) (end 69.5 94) (width 3) (layer B.Cu) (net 2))
 (segment (start 73 75.82) (end 73 90.5) (width 3) (layer B.Cu) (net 2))
 (segment (start 44.32 75.32) (end 26 75.32) (width 3) (layer B.Cu) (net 2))
 (segment (start 63 94) (end 44.32 75.32) (width 3) (layer B.Cu) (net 2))
 (segment (start 69.5 94) (end 63 94) (width 3) (layer B.Cu) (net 2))
 (segment (start 90.06 77) (end 90 77.06) (width 1.5) (layer B.Cu) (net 2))
 (segment (start 102.92 77) (end 90.06 77) (width 1.5) (layer B.Cu) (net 2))
 (segment (start 82.06 77.06) (end 80.82 75.82) (width 1.5) (layer B.Cu) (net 2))
 (segment (start 90 77.06) (end 82.06 77.06) (width 1.5) (layer B.Cu) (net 2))
 (segment (start 68 29) (end 68 34) (width 3) (layer B.Cu) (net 2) (status 1000000))
 (segment (start 63 24) (end 68 29) (width 3) (layer B.Cu) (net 2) (status 1000000))
 (segment (start 42 24) (end 63 24) (width 3) (layer B.Cu) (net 2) (status 1000000))
 (segment (start 42 24) (end 42 36) (width 3) (layer B.Cu) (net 2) (status 1000000))
 (segment (start 36 42) (end 42 36) (width 3) (layer B.Cu) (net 2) (status 1000000))
 (segment (start 36 46) (end 36 42) (width 3) (layer B.Cu) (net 2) (status 1000000))
 (segment (start 72 112) (end 72 110) (width 0.75) (layer F.Cu) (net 12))
 (segment (start 71 113) (end 72 112) (width 0.75) (layer F.Cu) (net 12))
 (segment (start 40.5 101) (end 40.5 110.5) (width 0.75) (layer F.Cu) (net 12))
 (segment (start 43 113) (end 43.5 113) (width 0.75) (layer F.Cu) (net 12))
 (segment (start 46 99.46) (end 42.04 99.46) (width 0.75) (layer F.Cu) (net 12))
 (segment (start 40.5 110.5) (end 43 113) (width 0.75) (layer F.Cu) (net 12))
 (segment (start 43.5 113) (end 71 113) (width 0.75) (layer F.Cu) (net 12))
 (segment (start 42.04 99.46) (end 40.5 101) (width 0.75) (layer F.Cu) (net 12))
 (segment (start 77 106) (end 77 110) (width 0.75) (layer F.Cu) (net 9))
 (segment (start 75.75 104.75) (end 77 106) (width 0.75) (layer F.Cu) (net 9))
 (segment (start 68.75 104.75) (end 75.75 104.75) (width 0.75) (layer F.Cu) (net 9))
 (segment (start 61.5 112) (end 68.75 104.75) (width 0.75) (layer F.Cu) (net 9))
 (segment (start 52 112) (end 61.5 112) (width 0.75) (layer F.Cu) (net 9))
 (segment (start 50.5 110.5) (end 52 112) (width 0.75) (layer F.Cu) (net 9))
 (segment (start 50.5 101) (end 50.5 110.5) (width 0.75) (layer F.Cu) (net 9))
 (segment (start 52.04 99.46) (end 50.5 101) (width 0.75) (layer F.Cu) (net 9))
 (segment (start 56 99.46) (end 52.04 99.46) (width 0.75) (layer F.Cu) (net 9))
 (segment (start 74.5 111.5) (end 74.5 110) (width 0.75) (layer F.Cu) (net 13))
 (segment (start 72.04999 113.95001) (end 74.5 111.5) (width 0.75) (layer F.Cu) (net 13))
 (segment (start 33.95001 113.95001) (end 34.95001 113.95001) (width 0.75) (layer F.Cu) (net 13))
 (segment (start 30.5 101) (end 30.5 110.5) (width 0.75) (layer F.Cu) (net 13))
 (segment (start 32.04 99.46) (end 30.5 101) (width 0.75) (layer F.Cu) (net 13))
 (segment (start 36 99.46) (end 32.04 99.46) (width 0.75) (layer F.Cu) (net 13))
 (segment (start 34.95001 113.95001) (end 72.04999 113.95001) (width 0.75) (layer F.Cu) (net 13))
 (segment (start 30.5 110.5) (end 33.95001 113.95001) (width 0.75) (layer F.Cu) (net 13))
 (segment (start 70.5 58) (end 73 55.5) (width 3) (layer B.Cu) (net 4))
 (segment (start 59 58) (end 70.5 58) (width 3) (layer B.Cu) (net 4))
 (segment (start 57.5 59.5) (end 59 58) (width 3) (layer B.Cu) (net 4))
 (segment (start 57.5 64.5) (end 57.5 59.5) (width 3) (layer B.Cu) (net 4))
 (segment (start 87.5 70) (end 73 55.5) (width 0.75) (layer F.Cu) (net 4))
 (segment (start 105.84 71.25) (end 88.75 71.25) (width 0.75) (layer F.Cu) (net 4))
 (segment (start 86.875 69.375) (end 73 55.5) (width 0.75) (layer F.Cu) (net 4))
 (segment (start 88.75 71.25) (end 86.875 69.375) (width 0.75) (layer F.Cu) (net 4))
 (segment (start 73 24) (end 77.27499 28.27499) (width 3) (layer B.Cu) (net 4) (status 1000000))
 (segment (start 77.27499 51.22501) (end 73 55.5) (width 3) (layer B.Cu) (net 4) (status 1000000))
 (segment (start 77.27499 28.27499) (end 77.27499 51.22501) (width 3) (layer B.Cu) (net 4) (status 1000000))
 (segment (start 28 87) (end 42 87) (width 3) (layer B.Cu) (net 6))
 (segment (start 21.72501 80.72501) (end 28 87) (width 3) (layer B.Cu) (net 6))
 (segment (start 21.72501 59.27499) (end 21.72501 80.72501) (width 3) (layer B.Cu) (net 6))
 (segment (start 26 55) (end 21.72501 59.27499) (width 3) (layer B.Cu) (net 6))
 (segment (start 42 81) (end 41.5 80.5) (width 3) (layer B.Cu) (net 6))
 (segment (start 42 87) (end 42 81) (width 3) (layer B.Cu) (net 6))
 (segment (start 24 45) (end 26 47) (width 3) (layer B.Cu) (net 6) (status 1000000))
 (segment (start 24 40) (end 24 45) (width 3) (layer B.Cu) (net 6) (status 1000000))
 (segment (start 26 55) (end 26 47) (width 3) (layer B.Cu) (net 6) (status 1000000))
 (segment (start 44.688542 104.54) (end 46 104.54) (width 0.75) (layer B.Cu) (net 1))
 (segment (start 36 104.54) (end 44.688542 104.54) (width 0.75) (layer B.Cu) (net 1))
 (segment (start 108 77) (end 108 78.5) (width 0.75) (layer F.Cu) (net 1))
 (segment (start 108 78.5) (end 105.5 81) (width 0.75) (layer F.Cu) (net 1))
 (segment (start 46 104.54) (end 56 104.54) (width 0.75) (layer B.Cu) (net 1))
 (segment (start 56 104.54) (end 63.96 104.54) (width 0.75) (layer F.Cu) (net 1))
 (segment (start 100.5 81) (end 105.5 81) (width 0.75) (layer F.Cu) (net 1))
 (segment (start 96.94 84.56) (end 100.5 81) (width 0.75) (layer F.Cu) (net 1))
 (segment (start 83.94 84.56) (end 63.96 104.54) (width 0.75) (layer F.Cu) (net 1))
 (segment (start 96.94 84.56) (end 83.94 84.56) (width 0.75) (layer F.Cu) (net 1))
 (segment (start 108 84.62) (end 113.46 84.62) (width 0.75) (layer F.Cu) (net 7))
 (segment (start 101.5 95) (end 96.5 95) (width 0.75) (layer F.Cu) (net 8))
 (segment (start 101.5 95) (end 101.5 90.5) (width 0.75) (layer F.Cu) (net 8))
 (segment (start 102.92 89.08) (end 102.92 84.62) (width 0.75) (layer F.Cu) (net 8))
 (segment (start 101.5 90.5) (end 102.92 89.08) (width 0.75) (layer F.Cu) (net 8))
 (segment (start 111.5 95) (end 116.5 95) (width 0.75) (layer F.Cu) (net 21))
 (segment (start 119.5 95) (end 116.5 95) (width 0.75) (layer F.Cu) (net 21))
 (segment (start 122 92.5) (end 119.5 95) (width 0.75) (layer F.Cu) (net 21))
 (segment (start 124 88.5) (end 122 90.5) (width 0.75) (layer F.Cu) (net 21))
 (segment (start 122 90.5) (end 122 92.5) (width 0.75) (layer F.Cu) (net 21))
 (segment (start 127.5 88.5) (end 124 88.5) (width 0.75) (layer F.Cu) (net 21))
 (segment (start 111.5 108) (end 116.5 108) (width 0.75) (layer F.Cu) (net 20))
 (segment (start 127.5 104.5) (end 124 104.5) (width 0.75) (layer F.Cu) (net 20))
 (segment (start 120.5 108) (end 116.5 108) (width 0.75) (layer F.Cu) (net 20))
 (segment (start 124 104.5) (end 120.5 108) (width 0.75) (layer F.Cu) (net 20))
 (segment (start 101.5 108) (end 96.5 108) (width 0.75) (layer F.Cu) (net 18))
 (segment (start 96.5 108) (end 89 108) (width 0.75) (layer F.Cu) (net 18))
 (segment (start 87 110) (end 82 110) (width 0.75) (layer F.Cu) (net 18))
 (segment (start 89 108) (end 87 110) (width 0.75) (layer F.Cu) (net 18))
 (segment (start 79.5 106) (end 84 101.5) (width 0.75) (layer F.Cu) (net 19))
 (segment (start 79.5 110) (end 79.5 106) (width 0.75) (layer F.Cu) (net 19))
 (segment (start 127.5 96.5) (end 124 96.5) (width 0.75) (layer F.Cu) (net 19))
 (segment (start 124 96.5) (end 119 101.5) (width 0.75) (layer F.Cu) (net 19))
 (segment (start 84 101.5) (end 119 101.5) (width 0.75) (layer F.Cu) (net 19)))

